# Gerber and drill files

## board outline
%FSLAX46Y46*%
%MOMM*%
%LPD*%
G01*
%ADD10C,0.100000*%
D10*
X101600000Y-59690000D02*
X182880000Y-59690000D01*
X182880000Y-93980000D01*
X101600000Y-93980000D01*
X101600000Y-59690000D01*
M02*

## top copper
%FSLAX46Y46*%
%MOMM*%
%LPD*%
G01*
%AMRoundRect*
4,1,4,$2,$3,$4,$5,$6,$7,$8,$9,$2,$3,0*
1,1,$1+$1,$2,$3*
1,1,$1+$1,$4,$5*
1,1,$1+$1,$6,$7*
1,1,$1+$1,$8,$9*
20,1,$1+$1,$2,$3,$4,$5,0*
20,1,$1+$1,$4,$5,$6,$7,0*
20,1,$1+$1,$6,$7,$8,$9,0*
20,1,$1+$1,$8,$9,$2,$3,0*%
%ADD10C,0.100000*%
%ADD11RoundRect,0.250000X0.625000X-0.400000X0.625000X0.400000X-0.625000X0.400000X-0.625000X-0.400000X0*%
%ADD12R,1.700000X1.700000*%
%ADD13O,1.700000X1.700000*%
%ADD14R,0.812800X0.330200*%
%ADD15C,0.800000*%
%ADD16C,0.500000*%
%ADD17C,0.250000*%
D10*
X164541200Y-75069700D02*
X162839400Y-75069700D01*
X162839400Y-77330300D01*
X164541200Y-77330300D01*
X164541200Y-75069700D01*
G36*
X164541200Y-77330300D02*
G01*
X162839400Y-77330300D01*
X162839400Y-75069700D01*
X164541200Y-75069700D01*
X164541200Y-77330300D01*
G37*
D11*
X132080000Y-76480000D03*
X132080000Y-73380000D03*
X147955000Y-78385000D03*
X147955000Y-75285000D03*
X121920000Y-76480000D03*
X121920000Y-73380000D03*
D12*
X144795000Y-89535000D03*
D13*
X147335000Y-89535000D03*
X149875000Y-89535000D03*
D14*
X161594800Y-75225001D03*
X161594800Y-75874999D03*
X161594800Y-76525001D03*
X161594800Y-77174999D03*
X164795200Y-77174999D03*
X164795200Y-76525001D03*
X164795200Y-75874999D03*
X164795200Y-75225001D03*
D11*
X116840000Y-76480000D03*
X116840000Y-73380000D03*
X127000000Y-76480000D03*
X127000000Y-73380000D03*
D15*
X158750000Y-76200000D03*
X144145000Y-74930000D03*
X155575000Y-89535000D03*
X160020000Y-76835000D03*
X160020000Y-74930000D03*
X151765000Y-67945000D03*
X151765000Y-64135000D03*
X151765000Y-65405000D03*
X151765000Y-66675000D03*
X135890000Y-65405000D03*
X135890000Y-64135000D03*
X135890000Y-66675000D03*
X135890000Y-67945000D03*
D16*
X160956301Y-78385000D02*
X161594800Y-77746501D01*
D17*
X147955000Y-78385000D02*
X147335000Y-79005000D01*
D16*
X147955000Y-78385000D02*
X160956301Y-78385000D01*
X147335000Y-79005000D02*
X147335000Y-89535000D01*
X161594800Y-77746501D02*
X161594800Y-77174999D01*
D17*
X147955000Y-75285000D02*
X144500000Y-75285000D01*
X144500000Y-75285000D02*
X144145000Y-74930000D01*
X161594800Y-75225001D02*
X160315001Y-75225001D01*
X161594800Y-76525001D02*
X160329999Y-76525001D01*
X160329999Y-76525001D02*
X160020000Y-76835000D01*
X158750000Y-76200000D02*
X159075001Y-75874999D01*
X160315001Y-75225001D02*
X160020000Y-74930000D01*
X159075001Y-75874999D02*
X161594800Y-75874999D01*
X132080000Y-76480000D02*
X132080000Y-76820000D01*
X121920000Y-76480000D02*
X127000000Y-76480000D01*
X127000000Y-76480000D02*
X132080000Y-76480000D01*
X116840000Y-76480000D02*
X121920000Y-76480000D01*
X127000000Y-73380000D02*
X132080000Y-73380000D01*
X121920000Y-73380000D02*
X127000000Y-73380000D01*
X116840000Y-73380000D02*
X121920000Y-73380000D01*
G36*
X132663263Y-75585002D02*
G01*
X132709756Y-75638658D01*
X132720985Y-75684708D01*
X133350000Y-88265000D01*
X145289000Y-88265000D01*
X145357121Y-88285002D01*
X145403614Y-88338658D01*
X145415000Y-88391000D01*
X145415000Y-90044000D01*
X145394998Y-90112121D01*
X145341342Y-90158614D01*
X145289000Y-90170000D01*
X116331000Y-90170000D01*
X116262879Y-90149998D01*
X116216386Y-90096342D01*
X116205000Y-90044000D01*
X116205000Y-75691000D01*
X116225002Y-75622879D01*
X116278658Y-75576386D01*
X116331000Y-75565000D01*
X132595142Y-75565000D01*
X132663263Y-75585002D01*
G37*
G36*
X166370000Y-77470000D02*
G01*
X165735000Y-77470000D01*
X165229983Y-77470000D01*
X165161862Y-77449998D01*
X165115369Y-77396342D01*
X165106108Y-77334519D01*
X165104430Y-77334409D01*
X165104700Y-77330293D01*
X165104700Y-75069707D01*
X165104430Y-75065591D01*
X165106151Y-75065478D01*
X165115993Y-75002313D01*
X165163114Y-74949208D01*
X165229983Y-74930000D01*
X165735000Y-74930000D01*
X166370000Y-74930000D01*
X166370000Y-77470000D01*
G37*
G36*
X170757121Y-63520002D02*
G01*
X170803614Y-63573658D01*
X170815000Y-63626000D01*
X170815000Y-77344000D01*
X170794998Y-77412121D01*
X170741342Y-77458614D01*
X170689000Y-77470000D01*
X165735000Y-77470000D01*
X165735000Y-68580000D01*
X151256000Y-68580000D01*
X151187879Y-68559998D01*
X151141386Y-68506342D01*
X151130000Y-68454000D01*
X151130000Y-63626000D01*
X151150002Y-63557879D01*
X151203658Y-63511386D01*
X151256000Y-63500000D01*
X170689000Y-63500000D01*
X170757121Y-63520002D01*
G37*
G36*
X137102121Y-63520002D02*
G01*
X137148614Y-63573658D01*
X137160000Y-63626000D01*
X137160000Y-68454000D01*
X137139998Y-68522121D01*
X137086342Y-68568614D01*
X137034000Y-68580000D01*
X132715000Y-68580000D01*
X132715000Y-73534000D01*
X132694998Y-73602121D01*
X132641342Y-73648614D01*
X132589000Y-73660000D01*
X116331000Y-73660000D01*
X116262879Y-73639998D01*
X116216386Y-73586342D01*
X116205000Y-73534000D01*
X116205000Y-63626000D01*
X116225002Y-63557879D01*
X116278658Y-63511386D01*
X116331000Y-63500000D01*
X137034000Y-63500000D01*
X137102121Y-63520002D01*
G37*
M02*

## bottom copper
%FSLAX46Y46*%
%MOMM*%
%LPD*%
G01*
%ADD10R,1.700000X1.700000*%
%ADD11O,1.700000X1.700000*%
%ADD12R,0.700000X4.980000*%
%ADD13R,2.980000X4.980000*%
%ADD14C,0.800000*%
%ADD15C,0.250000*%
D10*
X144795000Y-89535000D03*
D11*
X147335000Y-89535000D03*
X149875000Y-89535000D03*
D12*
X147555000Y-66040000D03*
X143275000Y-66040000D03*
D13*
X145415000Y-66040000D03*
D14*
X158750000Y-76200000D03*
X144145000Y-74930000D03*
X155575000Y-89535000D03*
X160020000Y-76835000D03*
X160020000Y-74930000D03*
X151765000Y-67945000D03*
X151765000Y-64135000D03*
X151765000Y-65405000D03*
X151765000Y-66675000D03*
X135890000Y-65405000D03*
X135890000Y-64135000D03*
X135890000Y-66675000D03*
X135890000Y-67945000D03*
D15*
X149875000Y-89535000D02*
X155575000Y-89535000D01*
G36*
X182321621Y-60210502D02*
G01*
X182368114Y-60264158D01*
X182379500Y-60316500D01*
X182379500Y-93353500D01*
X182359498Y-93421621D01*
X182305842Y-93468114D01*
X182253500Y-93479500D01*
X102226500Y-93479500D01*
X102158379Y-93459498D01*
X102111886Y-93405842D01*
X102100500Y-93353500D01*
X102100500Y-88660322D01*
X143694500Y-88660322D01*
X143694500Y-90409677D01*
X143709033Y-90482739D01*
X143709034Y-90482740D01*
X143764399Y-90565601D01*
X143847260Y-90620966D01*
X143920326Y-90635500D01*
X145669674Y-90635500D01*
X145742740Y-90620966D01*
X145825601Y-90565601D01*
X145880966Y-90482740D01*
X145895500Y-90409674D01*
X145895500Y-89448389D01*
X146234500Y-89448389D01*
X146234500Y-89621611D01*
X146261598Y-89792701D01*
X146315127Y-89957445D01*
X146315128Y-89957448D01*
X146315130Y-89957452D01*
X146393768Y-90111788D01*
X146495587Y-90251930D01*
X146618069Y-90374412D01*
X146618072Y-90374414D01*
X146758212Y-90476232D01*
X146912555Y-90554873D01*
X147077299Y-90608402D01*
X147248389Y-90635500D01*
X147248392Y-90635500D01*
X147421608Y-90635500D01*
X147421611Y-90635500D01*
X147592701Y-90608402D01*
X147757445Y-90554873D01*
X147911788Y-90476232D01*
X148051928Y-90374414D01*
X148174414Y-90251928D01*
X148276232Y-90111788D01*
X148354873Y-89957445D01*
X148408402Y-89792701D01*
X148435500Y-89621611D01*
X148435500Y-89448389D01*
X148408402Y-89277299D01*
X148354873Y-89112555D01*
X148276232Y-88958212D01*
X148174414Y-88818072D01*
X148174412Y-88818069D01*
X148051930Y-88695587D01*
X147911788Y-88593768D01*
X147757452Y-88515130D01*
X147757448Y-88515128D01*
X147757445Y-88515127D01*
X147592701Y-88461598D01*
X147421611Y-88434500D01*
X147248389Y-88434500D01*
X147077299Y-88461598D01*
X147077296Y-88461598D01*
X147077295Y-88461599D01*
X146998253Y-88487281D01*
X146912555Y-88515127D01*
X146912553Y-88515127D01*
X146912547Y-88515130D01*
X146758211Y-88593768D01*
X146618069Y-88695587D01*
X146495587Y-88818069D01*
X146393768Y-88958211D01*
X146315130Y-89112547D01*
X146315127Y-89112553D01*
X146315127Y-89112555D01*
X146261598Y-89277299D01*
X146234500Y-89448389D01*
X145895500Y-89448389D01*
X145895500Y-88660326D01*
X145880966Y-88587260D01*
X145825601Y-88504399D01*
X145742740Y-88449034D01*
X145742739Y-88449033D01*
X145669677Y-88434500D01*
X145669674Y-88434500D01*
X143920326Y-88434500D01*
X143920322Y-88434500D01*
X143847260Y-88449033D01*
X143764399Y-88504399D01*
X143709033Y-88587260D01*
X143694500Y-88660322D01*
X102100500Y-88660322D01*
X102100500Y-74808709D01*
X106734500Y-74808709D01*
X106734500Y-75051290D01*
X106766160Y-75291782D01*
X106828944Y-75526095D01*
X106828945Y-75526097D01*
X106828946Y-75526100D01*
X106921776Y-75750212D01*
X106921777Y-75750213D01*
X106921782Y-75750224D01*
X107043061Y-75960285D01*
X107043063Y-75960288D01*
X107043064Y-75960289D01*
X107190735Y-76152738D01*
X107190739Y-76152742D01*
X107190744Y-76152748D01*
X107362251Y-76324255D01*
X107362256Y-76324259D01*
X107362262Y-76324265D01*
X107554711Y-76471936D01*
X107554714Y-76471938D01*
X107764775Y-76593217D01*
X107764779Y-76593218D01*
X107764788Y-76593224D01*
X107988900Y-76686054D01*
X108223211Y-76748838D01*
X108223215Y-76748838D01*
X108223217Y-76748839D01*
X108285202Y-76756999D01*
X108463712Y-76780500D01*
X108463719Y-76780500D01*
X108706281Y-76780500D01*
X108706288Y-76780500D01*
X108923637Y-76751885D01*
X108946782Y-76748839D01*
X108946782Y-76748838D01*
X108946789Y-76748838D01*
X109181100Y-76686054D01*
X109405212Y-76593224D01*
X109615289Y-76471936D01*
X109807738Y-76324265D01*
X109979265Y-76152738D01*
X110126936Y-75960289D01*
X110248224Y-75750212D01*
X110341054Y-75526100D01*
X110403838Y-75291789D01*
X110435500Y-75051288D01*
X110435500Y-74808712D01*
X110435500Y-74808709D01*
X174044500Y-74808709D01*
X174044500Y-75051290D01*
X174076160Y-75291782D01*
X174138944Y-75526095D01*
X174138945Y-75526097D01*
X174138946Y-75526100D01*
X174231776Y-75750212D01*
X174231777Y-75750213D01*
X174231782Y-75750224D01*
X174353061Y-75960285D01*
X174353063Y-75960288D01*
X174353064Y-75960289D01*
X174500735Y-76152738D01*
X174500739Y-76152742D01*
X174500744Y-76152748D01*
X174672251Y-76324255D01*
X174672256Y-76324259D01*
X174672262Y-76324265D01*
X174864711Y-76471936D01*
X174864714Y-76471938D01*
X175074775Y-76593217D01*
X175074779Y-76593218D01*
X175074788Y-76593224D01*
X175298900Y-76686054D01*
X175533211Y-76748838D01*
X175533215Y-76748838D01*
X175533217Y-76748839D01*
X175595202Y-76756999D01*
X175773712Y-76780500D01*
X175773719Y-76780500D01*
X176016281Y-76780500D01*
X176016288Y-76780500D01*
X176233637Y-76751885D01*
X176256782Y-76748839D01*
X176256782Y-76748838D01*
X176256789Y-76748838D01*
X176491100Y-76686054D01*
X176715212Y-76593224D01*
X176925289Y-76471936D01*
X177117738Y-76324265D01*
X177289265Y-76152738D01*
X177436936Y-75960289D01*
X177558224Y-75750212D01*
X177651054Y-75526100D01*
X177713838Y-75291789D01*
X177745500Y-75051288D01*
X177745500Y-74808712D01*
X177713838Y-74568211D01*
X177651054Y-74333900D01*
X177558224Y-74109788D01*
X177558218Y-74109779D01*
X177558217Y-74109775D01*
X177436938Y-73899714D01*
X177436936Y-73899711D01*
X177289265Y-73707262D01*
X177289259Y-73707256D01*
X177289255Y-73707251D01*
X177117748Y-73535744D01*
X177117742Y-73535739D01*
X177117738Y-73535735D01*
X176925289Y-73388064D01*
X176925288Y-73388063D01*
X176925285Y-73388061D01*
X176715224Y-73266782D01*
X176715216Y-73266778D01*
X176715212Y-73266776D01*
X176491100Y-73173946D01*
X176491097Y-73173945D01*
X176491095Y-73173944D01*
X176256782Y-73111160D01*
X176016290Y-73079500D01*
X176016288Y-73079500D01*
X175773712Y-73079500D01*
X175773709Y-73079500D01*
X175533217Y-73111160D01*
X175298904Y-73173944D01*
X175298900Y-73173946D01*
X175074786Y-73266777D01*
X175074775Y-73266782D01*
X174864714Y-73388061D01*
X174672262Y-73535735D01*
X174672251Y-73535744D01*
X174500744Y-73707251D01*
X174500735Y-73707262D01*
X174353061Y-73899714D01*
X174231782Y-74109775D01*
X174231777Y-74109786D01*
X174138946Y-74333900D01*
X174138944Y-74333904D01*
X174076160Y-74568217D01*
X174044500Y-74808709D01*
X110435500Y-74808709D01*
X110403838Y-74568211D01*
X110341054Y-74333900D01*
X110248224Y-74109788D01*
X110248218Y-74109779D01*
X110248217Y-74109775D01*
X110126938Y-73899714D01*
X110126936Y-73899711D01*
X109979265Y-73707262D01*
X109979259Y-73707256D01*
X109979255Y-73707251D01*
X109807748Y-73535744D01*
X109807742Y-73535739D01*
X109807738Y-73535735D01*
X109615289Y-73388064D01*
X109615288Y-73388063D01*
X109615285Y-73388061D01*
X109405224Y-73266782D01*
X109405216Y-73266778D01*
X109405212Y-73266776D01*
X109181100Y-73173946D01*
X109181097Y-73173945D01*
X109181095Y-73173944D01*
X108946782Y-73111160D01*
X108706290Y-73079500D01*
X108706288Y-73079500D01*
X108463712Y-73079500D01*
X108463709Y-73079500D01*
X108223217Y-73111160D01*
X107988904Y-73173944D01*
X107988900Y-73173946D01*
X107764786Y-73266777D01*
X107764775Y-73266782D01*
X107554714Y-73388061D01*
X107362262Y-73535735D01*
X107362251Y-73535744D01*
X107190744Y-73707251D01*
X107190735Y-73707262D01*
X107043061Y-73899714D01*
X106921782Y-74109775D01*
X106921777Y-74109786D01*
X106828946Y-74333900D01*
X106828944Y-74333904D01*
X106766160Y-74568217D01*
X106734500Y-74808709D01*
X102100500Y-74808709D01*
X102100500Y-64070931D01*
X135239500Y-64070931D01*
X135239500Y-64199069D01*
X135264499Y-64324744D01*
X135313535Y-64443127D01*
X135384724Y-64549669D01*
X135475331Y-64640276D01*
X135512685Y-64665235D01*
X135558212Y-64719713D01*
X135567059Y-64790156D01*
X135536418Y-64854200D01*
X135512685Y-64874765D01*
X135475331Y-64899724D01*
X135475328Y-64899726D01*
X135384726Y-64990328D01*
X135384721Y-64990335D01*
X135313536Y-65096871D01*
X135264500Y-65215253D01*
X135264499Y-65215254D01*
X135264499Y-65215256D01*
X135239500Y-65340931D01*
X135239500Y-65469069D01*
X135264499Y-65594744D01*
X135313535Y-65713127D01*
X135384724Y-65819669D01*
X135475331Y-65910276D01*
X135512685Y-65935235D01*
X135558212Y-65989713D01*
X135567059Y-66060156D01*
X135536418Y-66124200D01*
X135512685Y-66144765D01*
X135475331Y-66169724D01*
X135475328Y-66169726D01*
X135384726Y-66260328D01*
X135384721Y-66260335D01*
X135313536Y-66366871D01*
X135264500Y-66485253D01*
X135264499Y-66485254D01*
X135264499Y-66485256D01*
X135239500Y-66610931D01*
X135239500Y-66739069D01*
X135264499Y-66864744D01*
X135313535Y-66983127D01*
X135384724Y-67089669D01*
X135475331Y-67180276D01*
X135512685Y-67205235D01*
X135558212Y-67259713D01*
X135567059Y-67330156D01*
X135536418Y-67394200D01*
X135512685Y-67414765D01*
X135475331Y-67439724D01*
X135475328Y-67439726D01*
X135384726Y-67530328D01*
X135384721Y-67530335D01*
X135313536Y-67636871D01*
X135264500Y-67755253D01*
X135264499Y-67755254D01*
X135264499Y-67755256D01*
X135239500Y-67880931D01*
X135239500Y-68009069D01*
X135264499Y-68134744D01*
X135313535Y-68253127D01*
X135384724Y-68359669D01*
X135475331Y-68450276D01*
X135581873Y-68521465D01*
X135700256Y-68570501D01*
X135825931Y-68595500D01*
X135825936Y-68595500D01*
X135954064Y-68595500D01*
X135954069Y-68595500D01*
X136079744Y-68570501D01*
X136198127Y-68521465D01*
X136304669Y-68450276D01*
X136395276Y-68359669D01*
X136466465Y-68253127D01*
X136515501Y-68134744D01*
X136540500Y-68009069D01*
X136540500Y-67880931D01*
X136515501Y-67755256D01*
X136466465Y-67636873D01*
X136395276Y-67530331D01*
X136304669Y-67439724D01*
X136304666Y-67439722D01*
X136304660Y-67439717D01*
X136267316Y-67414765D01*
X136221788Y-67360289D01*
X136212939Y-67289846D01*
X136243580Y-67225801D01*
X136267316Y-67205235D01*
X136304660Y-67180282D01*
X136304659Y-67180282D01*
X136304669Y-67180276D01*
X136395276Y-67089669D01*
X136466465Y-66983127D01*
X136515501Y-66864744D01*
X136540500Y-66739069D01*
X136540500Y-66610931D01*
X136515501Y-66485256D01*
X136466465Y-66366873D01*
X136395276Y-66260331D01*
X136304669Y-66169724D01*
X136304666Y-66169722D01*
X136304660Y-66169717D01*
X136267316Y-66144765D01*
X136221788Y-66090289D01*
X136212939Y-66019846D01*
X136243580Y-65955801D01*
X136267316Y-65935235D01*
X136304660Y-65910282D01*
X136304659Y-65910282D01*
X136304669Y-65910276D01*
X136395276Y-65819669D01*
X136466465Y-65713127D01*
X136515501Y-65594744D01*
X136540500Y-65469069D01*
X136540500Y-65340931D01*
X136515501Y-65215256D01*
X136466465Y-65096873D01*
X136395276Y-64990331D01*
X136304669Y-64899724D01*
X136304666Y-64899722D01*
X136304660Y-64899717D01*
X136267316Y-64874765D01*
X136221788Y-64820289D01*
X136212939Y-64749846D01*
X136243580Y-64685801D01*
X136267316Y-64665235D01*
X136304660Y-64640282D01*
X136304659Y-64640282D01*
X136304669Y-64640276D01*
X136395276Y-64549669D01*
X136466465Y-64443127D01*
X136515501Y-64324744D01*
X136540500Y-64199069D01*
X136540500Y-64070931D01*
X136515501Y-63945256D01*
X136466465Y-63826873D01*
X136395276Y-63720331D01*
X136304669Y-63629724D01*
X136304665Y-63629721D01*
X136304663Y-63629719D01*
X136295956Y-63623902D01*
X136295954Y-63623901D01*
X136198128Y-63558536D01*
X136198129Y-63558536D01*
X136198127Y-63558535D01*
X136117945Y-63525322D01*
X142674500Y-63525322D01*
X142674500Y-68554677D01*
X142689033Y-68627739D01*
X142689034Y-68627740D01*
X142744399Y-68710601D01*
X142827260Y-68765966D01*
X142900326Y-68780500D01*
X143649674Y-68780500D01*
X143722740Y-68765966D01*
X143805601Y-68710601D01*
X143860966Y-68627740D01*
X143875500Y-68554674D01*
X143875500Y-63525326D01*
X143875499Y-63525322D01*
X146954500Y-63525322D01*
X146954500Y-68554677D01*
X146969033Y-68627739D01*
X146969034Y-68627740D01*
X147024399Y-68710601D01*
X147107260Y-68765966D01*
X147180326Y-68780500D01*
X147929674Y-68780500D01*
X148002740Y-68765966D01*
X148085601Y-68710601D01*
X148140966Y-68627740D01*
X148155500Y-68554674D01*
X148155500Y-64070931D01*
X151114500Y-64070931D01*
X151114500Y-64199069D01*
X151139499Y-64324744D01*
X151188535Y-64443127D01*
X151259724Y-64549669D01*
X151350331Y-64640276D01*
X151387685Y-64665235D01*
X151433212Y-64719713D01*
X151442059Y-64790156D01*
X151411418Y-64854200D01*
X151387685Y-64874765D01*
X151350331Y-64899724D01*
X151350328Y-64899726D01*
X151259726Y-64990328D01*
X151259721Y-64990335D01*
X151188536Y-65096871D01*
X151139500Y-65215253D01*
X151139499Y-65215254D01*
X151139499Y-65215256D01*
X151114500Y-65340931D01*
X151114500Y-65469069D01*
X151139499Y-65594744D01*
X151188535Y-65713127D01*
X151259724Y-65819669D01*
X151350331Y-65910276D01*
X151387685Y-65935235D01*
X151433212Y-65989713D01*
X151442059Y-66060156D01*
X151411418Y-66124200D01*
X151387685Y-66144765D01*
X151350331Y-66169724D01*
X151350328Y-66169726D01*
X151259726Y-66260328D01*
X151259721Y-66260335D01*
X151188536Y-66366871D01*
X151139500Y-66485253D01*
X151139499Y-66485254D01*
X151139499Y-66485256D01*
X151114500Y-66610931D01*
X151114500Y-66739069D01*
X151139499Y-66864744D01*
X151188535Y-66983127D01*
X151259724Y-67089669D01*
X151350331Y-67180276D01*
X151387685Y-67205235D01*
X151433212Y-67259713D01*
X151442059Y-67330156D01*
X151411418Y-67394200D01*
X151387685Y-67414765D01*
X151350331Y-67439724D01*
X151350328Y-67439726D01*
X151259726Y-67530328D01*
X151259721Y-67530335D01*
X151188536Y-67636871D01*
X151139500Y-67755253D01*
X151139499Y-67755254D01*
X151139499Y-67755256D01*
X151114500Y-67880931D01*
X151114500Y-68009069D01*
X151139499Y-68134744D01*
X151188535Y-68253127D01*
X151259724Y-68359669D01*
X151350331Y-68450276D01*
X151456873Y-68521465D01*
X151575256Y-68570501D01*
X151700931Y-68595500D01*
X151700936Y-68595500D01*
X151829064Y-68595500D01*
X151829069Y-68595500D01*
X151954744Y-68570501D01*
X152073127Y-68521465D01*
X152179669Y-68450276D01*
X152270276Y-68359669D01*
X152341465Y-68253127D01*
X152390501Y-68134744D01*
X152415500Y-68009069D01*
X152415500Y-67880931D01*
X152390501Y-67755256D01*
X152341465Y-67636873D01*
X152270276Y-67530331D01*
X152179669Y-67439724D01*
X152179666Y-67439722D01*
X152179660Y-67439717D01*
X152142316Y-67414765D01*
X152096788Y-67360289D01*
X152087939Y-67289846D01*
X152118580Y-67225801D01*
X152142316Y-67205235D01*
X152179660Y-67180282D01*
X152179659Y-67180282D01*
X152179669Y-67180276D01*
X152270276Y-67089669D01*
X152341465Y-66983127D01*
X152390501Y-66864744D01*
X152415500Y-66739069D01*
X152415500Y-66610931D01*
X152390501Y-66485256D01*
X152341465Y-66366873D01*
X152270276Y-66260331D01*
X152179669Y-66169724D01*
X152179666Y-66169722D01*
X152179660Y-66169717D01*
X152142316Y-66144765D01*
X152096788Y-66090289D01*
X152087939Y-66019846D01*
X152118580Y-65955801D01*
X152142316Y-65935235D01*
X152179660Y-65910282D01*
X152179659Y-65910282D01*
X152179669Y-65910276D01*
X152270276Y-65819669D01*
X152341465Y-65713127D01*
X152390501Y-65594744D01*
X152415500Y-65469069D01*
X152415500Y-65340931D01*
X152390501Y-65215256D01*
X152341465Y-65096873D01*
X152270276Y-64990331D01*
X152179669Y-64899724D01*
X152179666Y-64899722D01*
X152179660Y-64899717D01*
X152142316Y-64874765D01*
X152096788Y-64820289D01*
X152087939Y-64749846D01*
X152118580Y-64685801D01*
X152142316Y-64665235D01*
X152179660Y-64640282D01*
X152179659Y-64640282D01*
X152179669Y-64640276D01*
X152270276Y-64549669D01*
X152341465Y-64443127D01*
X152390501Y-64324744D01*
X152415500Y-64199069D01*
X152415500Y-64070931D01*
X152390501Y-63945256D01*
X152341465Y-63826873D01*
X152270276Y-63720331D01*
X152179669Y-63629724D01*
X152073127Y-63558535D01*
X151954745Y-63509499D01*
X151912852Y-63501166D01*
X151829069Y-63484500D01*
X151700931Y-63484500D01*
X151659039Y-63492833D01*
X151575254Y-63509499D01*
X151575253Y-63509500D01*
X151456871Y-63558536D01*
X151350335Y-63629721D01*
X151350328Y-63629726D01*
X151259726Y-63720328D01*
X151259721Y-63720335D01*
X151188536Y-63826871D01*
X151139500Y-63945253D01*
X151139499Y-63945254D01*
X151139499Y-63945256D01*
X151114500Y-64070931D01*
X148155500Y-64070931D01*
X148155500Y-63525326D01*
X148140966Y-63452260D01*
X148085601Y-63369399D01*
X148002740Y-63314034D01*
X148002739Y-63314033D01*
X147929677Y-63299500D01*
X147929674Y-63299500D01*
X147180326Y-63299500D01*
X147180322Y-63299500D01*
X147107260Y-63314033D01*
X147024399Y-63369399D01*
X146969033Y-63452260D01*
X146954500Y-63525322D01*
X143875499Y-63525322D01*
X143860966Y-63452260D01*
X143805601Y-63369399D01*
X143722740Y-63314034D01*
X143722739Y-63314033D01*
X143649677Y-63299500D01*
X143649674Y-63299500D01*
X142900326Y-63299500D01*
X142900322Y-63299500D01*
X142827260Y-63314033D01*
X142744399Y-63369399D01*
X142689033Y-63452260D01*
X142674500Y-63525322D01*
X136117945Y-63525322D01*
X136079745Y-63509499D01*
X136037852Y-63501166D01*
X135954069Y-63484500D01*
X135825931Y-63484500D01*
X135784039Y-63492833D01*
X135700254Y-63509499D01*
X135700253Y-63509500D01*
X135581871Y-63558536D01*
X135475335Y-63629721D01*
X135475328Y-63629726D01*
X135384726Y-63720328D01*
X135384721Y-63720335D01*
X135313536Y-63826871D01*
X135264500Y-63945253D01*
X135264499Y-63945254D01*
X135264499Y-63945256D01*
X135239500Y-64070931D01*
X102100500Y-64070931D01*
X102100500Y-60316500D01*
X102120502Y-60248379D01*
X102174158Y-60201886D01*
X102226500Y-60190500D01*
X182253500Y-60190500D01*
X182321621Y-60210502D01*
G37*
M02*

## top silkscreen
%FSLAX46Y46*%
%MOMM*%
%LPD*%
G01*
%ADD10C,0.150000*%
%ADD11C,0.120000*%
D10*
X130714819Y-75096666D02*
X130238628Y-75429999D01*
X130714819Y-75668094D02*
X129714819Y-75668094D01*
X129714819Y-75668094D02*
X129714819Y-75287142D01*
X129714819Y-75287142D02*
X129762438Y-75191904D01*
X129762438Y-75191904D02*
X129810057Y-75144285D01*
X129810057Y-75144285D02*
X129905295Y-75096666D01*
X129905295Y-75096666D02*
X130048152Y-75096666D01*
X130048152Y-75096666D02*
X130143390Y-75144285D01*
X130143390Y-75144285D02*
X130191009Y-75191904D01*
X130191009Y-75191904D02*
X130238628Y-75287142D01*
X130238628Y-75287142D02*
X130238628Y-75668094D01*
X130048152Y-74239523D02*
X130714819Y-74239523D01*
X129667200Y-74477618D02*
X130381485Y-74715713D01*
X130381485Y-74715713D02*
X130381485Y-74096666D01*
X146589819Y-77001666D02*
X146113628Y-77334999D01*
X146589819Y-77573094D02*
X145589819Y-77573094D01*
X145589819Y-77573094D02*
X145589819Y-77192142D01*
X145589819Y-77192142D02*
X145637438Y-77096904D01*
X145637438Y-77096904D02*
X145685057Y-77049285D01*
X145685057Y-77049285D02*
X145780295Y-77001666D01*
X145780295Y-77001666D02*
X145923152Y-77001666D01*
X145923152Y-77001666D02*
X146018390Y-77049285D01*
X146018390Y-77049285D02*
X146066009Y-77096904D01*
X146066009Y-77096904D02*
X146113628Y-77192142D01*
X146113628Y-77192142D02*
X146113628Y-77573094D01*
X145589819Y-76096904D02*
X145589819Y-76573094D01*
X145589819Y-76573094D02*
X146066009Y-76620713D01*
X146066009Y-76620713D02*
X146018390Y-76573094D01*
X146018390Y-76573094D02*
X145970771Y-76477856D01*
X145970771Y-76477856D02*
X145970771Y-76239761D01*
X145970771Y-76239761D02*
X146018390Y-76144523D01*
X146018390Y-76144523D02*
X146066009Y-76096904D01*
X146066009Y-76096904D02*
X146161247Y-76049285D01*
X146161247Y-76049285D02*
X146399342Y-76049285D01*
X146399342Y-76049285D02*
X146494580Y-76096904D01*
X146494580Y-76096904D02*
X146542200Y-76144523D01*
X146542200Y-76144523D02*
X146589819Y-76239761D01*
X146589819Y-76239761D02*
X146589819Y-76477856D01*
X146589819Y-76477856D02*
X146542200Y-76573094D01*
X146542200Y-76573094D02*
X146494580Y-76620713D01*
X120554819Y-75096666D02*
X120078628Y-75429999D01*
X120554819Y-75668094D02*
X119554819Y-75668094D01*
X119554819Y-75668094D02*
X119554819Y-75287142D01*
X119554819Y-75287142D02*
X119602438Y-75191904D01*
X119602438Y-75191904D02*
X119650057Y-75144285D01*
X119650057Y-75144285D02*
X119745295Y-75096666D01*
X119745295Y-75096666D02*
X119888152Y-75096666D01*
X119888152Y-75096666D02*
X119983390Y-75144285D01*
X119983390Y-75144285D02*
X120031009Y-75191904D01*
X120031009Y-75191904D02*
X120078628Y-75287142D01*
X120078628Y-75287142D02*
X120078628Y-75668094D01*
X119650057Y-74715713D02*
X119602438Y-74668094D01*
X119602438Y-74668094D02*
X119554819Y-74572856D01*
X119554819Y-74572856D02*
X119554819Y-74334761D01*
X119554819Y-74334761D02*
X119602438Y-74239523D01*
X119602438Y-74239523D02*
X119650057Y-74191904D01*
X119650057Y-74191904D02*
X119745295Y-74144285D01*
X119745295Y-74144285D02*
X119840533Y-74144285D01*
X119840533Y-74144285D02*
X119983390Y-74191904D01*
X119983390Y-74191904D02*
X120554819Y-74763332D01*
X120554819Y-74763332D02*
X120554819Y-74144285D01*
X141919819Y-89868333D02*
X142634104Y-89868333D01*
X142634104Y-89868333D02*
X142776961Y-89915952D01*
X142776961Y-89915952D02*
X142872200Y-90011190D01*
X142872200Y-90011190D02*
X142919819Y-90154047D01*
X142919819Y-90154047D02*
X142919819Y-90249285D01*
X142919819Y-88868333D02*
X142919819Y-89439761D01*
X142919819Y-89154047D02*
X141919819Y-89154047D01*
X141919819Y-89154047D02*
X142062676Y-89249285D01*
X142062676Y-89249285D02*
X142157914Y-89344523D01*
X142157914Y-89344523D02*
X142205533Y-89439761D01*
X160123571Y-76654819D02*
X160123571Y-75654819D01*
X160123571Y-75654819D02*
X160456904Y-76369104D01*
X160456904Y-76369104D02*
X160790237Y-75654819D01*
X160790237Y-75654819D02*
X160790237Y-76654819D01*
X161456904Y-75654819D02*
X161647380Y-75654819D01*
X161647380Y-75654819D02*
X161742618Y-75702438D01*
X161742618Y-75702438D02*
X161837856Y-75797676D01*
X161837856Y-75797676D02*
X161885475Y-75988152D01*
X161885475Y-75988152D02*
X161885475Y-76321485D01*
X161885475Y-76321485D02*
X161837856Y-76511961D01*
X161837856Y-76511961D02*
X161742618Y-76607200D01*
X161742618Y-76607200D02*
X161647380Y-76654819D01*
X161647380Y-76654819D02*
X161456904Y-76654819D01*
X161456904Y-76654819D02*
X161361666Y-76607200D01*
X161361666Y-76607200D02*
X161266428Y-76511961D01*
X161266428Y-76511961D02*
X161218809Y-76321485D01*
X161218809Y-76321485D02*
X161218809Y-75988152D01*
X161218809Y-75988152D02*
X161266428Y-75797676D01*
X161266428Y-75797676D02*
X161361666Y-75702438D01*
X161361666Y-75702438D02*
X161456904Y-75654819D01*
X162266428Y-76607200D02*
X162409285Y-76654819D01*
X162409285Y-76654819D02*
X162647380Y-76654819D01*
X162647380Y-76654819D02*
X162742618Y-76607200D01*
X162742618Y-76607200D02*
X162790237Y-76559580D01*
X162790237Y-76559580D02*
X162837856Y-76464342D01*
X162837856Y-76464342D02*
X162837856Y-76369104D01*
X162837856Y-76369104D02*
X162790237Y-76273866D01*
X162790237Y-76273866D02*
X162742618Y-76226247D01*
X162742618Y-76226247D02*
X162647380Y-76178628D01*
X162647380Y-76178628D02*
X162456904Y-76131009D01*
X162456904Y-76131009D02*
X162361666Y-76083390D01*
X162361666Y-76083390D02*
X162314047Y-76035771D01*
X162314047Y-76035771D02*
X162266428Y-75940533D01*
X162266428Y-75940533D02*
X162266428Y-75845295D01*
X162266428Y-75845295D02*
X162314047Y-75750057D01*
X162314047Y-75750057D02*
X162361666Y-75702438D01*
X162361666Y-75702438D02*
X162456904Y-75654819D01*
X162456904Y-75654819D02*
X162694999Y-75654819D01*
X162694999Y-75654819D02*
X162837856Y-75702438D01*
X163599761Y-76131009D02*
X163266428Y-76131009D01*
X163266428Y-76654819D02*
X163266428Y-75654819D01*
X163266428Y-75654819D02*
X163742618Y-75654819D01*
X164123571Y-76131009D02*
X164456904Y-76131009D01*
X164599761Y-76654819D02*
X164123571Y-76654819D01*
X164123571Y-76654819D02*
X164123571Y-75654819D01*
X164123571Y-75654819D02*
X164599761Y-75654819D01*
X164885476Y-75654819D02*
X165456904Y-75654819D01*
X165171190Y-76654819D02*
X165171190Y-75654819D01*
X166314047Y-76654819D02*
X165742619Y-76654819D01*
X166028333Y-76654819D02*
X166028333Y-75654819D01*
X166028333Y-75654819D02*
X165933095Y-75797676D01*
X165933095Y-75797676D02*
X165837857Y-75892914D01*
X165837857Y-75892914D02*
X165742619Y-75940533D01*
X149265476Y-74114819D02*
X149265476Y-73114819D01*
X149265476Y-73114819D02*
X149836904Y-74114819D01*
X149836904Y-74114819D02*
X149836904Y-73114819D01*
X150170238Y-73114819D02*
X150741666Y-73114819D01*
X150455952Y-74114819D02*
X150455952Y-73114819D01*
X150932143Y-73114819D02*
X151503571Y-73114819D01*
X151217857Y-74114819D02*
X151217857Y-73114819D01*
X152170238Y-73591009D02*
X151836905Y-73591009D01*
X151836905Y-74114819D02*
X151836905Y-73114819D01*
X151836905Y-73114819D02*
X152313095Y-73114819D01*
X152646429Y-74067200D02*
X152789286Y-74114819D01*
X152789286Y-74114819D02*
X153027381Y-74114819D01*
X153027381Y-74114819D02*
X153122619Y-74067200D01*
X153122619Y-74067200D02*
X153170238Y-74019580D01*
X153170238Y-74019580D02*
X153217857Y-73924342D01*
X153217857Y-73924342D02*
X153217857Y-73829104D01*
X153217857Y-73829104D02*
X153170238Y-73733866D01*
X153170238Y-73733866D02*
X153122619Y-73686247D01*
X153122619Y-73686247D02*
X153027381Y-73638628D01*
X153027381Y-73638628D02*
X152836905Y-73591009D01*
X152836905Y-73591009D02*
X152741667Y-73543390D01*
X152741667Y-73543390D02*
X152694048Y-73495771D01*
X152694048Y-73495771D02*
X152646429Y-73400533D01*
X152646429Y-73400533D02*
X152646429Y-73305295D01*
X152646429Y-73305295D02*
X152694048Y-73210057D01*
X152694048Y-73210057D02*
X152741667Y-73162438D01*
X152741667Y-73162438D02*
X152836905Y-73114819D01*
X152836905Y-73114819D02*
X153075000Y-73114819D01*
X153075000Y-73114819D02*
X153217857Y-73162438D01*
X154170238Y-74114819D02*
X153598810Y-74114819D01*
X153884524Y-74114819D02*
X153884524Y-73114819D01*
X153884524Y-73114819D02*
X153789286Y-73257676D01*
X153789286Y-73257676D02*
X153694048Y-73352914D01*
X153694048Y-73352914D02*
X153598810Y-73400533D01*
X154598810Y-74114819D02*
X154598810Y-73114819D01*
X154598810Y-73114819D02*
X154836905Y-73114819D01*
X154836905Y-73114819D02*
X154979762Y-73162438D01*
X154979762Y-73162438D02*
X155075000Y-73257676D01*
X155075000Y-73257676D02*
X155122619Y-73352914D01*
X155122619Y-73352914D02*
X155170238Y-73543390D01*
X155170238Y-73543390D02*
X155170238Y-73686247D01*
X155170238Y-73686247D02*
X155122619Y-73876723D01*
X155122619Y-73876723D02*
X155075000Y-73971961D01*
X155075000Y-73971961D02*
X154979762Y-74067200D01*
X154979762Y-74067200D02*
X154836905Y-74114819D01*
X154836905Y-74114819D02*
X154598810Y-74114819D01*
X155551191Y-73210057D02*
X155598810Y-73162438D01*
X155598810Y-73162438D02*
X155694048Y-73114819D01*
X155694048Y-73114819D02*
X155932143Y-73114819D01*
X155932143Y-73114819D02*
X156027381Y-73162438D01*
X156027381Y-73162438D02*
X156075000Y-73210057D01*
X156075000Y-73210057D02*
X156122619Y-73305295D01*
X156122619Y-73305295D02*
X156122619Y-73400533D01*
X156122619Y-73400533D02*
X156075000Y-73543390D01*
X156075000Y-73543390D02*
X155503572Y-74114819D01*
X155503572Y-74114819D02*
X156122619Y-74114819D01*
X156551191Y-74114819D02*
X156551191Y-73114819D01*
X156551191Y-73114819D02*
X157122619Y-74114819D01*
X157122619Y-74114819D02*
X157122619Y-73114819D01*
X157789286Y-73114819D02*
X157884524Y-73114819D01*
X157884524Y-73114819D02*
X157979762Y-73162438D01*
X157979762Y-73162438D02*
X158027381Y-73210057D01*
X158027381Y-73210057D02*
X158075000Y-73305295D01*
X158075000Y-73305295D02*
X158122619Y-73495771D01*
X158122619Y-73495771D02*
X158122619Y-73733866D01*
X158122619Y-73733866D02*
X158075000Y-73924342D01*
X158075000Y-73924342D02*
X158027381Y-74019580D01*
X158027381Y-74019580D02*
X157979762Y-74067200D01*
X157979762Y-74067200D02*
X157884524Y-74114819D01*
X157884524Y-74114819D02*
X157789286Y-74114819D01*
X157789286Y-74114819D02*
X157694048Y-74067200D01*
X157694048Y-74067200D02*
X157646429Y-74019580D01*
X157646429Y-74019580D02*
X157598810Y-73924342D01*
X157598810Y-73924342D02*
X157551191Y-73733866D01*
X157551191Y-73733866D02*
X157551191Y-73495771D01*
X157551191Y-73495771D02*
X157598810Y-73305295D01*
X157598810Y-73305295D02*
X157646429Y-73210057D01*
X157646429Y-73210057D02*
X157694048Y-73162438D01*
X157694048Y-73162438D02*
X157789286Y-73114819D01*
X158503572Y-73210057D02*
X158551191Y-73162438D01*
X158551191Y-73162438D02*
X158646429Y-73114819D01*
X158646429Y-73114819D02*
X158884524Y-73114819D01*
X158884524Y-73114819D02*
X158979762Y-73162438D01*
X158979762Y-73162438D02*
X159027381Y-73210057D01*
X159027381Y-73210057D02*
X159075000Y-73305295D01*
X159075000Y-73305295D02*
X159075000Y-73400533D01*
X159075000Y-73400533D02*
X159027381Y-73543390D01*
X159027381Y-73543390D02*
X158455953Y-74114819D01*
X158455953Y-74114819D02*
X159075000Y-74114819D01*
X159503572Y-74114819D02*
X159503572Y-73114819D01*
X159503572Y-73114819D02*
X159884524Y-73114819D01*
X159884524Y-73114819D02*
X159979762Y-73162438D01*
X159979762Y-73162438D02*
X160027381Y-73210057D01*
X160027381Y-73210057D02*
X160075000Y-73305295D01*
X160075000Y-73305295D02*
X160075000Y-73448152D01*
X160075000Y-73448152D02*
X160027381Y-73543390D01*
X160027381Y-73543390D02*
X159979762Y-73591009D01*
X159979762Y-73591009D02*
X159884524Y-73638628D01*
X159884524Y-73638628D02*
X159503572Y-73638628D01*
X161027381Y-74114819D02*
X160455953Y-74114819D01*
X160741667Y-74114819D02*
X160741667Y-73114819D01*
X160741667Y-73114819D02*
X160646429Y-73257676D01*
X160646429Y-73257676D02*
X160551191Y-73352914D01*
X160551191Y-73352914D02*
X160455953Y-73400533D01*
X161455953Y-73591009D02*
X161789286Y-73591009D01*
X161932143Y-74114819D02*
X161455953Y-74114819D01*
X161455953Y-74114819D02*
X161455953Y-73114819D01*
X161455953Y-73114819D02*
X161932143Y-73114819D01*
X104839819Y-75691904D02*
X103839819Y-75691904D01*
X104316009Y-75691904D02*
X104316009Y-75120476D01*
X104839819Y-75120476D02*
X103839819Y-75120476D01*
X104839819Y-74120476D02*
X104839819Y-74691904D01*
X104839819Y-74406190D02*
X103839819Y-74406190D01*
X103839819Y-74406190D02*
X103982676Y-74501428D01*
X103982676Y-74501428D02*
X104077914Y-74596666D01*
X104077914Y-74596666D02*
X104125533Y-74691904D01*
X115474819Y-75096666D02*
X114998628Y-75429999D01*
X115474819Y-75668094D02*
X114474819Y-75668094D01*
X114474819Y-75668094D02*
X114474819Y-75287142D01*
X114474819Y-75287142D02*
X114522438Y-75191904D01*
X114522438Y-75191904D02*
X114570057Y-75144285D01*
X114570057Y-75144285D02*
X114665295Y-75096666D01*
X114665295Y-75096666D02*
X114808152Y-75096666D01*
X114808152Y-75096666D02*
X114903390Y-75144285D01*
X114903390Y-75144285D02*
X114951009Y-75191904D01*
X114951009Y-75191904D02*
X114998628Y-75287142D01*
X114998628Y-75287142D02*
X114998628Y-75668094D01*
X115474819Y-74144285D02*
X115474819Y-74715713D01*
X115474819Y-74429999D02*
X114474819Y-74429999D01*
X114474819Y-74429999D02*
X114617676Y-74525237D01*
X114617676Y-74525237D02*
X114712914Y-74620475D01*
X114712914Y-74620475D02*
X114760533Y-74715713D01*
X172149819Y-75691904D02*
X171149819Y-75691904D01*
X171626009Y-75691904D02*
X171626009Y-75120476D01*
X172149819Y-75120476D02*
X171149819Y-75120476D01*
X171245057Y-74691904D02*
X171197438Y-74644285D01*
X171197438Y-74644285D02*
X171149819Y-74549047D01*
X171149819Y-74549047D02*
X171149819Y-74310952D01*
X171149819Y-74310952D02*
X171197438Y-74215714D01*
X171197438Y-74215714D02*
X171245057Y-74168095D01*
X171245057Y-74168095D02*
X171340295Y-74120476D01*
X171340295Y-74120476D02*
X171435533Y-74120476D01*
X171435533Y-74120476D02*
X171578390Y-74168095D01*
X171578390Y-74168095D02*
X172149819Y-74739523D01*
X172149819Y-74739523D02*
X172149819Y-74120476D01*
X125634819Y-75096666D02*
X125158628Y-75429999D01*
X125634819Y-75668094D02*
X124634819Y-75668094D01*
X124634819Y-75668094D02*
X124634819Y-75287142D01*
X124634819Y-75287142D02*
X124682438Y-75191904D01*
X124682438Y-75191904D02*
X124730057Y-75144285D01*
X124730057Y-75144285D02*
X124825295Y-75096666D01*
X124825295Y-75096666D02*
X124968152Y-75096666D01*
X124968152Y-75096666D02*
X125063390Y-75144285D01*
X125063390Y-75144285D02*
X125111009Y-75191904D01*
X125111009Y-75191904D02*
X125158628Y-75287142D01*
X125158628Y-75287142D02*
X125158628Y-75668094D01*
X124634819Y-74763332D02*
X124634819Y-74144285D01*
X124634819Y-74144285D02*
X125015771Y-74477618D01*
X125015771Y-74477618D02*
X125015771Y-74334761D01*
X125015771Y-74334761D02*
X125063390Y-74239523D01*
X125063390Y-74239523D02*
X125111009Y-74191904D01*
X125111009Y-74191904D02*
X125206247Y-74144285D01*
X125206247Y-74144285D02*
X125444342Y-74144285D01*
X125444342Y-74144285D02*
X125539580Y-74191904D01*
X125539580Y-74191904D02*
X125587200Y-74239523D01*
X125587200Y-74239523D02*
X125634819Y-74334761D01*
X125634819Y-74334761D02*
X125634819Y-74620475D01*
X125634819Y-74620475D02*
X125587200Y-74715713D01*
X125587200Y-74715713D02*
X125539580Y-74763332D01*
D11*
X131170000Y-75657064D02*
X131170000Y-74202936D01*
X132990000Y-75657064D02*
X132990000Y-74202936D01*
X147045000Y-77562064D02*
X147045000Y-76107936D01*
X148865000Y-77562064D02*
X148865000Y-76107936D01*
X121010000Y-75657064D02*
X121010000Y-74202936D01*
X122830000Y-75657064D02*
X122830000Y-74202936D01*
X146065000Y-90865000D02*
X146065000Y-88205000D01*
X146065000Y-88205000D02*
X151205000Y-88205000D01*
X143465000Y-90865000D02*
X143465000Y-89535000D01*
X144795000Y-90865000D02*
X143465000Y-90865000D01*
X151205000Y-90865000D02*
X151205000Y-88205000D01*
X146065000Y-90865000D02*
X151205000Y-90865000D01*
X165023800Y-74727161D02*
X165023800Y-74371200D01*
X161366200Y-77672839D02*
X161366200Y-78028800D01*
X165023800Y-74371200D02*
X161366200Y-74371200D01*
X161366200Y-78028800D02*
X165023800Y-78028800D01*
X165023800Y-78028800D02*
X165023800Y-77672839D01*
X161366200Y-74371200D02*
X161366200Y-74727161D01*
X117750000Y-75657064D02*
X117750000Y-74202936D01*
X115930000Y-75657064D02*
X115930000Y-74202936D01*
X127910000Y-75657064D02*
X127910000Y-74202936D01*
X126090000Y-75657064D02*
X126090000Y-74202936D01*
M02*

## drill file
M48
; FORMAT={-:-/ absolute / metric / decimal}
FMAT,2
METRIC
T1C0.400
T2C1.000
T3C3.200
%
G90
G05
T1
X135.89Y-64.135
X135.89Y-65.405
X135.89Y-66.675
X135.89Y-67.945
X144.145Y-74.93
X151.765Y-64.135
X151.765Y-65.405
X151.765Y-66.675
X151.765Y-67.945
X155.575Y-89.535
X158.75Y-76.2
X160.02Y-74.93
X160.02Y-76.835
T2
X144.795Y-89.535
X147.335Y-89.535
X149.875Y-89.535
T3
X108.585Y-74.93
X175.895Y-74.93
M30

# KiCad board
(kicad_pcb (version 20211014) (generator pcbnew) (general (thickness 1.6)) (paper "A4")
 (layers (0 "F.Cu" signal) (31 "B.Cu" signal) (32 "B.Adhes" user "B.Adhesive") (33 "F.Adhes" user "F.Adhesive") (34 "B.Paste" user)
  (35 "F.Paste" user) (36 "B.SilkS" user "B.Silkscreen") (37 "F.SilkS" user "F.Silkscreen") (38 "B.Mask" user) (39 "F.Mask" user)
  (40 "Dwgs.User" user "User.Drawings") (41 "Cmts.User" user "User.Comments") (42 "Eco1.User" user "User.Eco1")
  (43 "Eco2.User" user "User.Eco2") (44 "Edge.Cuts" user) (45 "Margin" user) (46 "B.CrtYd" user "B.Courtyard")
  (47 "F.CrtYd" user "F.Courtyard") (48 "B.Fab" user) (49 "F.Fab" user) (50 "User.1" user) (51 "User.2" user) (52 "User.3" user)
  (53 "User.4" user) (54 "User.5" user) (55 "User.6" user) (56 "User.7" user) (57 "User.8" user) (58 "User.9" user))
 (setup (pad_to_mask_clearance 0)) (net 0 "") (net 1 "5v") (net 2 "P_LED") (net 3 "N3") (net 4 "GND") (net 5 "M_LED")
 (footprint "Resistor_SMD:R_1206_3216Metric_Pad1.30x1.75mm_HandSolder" (layer "F.Cu") (at 132.08 74.93 90)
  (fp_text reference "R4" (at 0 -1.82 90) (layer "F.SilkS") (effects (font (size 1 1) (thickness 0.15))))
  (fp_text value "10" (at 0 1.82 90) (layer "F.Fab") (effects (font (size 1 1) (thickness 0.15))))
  (fp_line (start -0.727064 -0.91) (end 0.727064 -0.91) (layer "F.SilkS") (width 0.12))
  (fp_line (start -0.727064 0.91) (end 0.727064 0.91) (layer "F.SilkS") (width 0.12))
  (pad "1" smd roundrect (at -1.55 0 90) (size 1.3 1.75) (layers "F.Cu" "F.Paste" "F.Mask") (roundrect_rratio 0.1923076923) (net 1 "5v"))
  (pad "2" smd roundrect (at 1.55 0 90) (size 1.3 1.75) (layers "F.Cu" "F.Paste" "F.Mask") (roundrect_rratio 0.1923076923) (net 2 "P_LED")))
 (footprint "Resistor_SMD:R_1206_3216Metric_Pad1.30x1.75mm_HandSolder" (layer "F.Cu") (at 147.955 76.835 90)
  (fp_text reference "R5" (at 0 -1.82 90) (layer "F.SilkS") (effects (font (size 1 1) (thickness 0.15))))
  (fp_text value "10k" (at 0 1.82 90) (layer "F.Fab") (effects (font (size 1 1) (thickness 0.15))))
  (fp_line (start -0.727064 -0.91) (end 0.727064 -0.91) (layer "F.SilkS") (width 0.12))
  (fp_line (start -0.727064 0.91) (end 0.727064 0.91) (layer "F.SilkS") (width 0.12))
  (pad "1" smd roundrect (at -1.55 0 90) (size 1.3 1.75) (layers "F.Cu" "F.Paste" "F.Mask") (roundrect_rratio 0.1923076923) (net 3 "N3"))
  (pad "2" smd roundrect (at 1.55 0 90) (size 1.3 1.75) (layers "F.Cu" "F.Paste" "F.Mask") (roundrect_rratio 0.1923076923) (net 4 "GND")))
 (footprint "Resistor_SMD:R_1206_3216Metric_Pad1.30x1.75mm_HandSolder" (layer "F.Cu") (at 121.92 74.93 90)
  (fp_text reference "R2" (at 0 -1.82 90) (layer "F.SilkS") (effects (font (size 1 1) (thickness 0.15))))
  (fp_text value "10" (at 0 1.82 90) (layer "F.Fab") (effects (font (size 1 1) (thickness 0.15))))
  (fp_line (start -0.727064 -0.91) (end 0.727064 -0.91) (layer "F.SilkS") (width 0.12))
  (fp_line (start -0.727064 0.91) (end 0.727064 0.91) (layer "F.SilkS") (width 0.12))
  (pad "1" smd roundrect (at -1.55 0 90) (size 1.3 1.75) (layers "F.Cu" "F.Paste" "F.Mask") (roundrect_rratio 0.1923076923) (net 1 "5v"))
  (pad "2" smd roundrect (at 1.55 0 90) (size 1.3 1.75) (layers "F.Cu" "F.Paste" "F.Mask") (roundrect_rratio 0.1923076923) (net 2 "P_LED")))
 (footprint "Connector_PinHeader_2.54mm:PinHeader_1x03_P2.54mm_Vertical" (layer "F.Cu") (at 144.795 89.535 90)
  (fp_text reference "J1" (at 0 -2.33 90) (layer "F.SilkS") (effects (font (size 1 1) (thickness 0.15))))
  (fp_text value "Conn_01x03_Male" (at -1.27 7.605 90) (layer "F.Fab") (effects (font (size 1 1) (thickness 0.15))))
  (fp_line (start -1.33 1.27) (end 1.33 1.27) (layer "F.SilkS") (width 0.12))
  (fp_line (start 1.33 1.27) (end 1.33 6.41) (layer "F.SilkS") (width 0.12))
  (fp_line (start -1.33 -1.33) (end 0 -1.33) (layer "F.SilkS") (width 0.12))
  (fp_line (start -1.33 0) (end -1.33 -1.33) (layer "F.SilkS") (width 0.12))
  (fp_line (start -1.33 6.41) (end 1.33 6.41) (layer "F.SilkS") (width 0.12))
  (fp_line (start -1.33 1.27) (end -1.33 6.41) (layer "F.SilkS") (width 0.12))
  (pad "1" thru_hole rect (at 0 0 90) (size 1.7 1.7) (drill 1) (layers *.Cu *.Mask) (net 1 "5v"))
  (pad "2" thru_hole oval (at 0 2.54 90) (size 1.7 1.7) (drill 1) (layers *.Cu *.Mask) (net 3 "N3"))
  (pad "3" thru_hole oval (at 0 5.08 90) (size 1.7 1.7) (drill 1) (layers *.Cu *.Mask) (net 4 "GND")))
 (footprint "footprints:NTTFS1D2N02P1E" (layer "F.Cu") (at 163.195 76.2)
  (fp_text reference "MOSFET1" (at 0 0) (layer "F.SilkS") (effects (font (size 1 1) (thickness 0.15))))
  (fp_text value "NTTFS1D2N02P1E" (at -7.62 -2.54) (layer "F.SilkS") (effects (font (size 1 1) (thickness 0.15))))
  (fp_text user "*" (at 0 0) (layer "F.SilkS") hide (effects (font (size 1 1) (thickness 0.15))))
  (fp_poly (pts (xy 1.3462 -1.1303) (xy -0.3556 -1.1303) (xy -0.3556 1.1303) (xy 1.3462 1.1303)) (layer "F.Cu") (width 0.1) (fill solid))
  (fp_line (start 1.8288 -1.472839) (end 1.8288 -1.8288) (layer "F.SilkS") (width 0.12))
  (fp_line (start -1.8288 1.472839) (end -1.8288 1.8288) (layer "F.SilkS") (width 0.12))
  (fp_line (start 1.8288 -1.8288) (end -1.8288 -1.8288) (layer "F.SilkS") (width 0.12))
  (fp_line (start -1.8288 1.8288) (end 1.8288 1.8288) (layer "F.SilkS") (width 0.12))
  (fp_line (start 1.8288 1.8288) (end 1.8288 1.472839) (layer "F.SilkS") (width 0.12))
  (fp_line (start -1.8288 -1.8288) (end -1.8288 -1.472839) (layer "F.SilkS") (width 0.12))
  (pad "1" smd rect (at -1.6002 -0.974999) (size 0.8128 0.3302) (layers "F.Cu" "F.Paste" "F.Mask") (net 4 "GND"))
  (pad "2" smd rect (at -1.6002 -0.325001) (size 0.8128 0.3302) (layers "F.Cu" "F.Paste" "F.Mask") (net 4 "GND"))
  (pad "3" smd rect (at -1.6002 0.325001) (size 0.8128 0.3302) (layers "F.Cu" "F.Paste" "F.Mask") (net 4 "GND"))
  (pad "4" smd rect (at -1.6002 0.974999) (size 0.8128 0.3302) (layers "F.Cu" "F.Paste" "F.Mask") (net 3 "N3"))
  (pad "5" smd rect (at 1.6002 0.974999) (size 0.8128 0.3302) (layers "F.Cu" "F.Paste" "F.Mask") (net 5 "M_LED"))
  (pad "6" smd rect (at 1.6002 0.325001) (size 0.8128 0.3302) (layers "F.Cu" "F.Paste" "F.Mask") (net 5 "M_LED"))
  (pad "7" smd rect (at 1.6002 -0.325001) (size 0.8128 0.3302) (layers "F.Cu" "F.Paste" "F.Mask") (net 5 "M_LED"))
  (pad "8" smd rect (at 1.6002 -0.974999) (size 0.8128 0.3302) (layers "F.Cu" "F.Paste" "F.Mask") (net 5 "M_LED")))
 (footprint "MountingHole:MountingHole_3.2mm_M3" (layer "F.Cu") (at 108.585 74.93 90)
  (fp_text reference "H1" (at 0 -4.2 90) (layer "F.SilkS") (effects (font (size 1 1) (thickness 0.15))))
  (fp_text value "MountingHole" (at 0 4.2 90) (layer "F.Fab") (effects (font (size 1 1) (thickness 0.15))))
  (pad "" np_thru_hole circle (at 0 0 90) (size 3.2 3.2) (drill 3.2) (layers *.Cu *.Mask)))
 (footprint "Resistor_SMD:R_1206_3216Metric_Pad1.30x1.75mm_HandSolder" (layer "F.Cu") (at 116.84 74.93 90)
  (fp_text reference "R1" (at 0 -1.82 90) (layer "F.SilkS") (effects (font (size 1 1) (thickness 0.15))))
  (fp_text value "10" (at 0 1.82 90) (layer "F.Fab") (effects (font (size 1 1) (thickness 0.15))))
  (fp_line (start -0.727064 0.91) (end 0.727064 0.91) (layer "F.SilkS") (width 0.12))
  (fp_line (start -0.727064 -0.91) (end 0.727064 -0.91) (layer "F.SilkS") (width 0.12))
  (pad "1" smd roundrect (at -1.55 0 90) (size 1.3 1.75) (layers "F.Cu" "F.Paste" "F.Mask") (roundrect_rratio 0.1923076923) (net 1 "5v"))
  (pad "2" smd roundrect (at 1.55 0 90) (size 1.3 1.75) (layers "F.Cu" "F.Paste" "F.Mask") (roundrect_rratio 0.1923076923) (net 2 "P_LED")))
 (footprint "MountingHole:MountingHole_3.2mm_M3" (layer "F.Cu") (at 175.895 74.93 90)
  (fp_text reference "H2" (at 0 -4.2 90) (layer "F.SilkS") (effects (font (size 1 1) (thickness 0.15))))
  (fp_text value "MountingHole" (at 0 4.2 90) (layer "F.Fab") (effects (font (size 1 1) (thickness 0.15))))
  (pad "" np_thru_hole circle (at 0 0 90) (size 3.2 3.2) (drill 3.2) (layers *.Cu *.Mask)))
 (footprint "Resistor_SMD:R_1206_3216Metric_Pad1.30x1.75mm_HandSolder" (layer "F.Cu") (at 127 74.93 90)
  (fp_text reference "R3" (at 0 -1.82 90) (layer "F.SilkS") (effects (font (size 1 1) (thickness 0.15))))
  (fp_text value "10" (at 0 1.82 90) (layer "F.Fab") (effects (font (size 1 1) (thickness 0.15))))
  (fp_line (start -0.727064 0.91) (end 0.727064 0.91) (layer "F.SilkS") (width 0.12))
  (fp_line (start -0.727064 -0.91) (end 0.727064 -0.91) (layer "F.SilkS") (width 0.12))
  (pad "1" smd roundrect (at -1.55 0 90) (size 1.3 1.75) (layers "F.Cu" "F.Paste" "F.Mask") (roundrect_rratio 0.1923076923) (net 1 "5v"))
  (pad "2" smd roundrect (at 1.55 0 90) (size 1.3 1.75) (layers "F.Cu" "F.Paste" "F.Mask") (roundrect_rratio 0.1923076923) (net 2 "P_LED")))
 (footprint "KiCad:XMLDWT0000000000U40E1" (layer "B.Cu") (at 145.415 66.04 180)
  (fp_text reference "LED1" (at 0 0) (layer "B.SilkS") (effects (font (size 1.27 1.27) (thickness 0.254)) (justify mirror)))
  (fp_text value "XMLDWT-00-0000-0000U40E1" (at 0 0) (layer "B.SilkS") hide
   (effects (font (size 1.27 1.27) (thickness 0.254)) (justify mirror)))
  (pad "1" smd rect locked (at -2.14 0 180) (size 0.7 4.98) (layers "B.Cu" "B.Paste" "B.Mask") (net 5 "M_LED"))
  (pad "2" smd rect locked (at 2.14 0 180) (size 0.7 4.98) (layers "B.Cu" "B.Paste" "B.Mask") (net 2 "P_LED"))
  (pad "3" smd rect locked (at 0 0 180) (size 2.98 4.98) (layers "B.Cu" "B.Paste" "B.Mask") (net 4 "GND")))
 (gr_rect (start 101.6 59.69) (end 182.88 93.98) (layer "Edge.Cuts") (width 0.1) (fill none))
 (segment (start 160.956301 78.385) (end 161.5948 77.746501) (width 0.5) (layer "F.Cu") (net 3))
 (segment (start 147.955 78.385) (end 147.335 79.005) (width 0.25) (layer "F.Cu") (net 3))
 (segment (start 147.955 78.385) (end 160.956301 78.385) (width 0.5) (layer "F.Cu") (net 3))
 (segment (start 147.335 79.005) (end 147.335 89.535) (width 0.5) (layer "F.Cu") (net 3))
 (segment (start 161.5948 77.746501) (end 161.5948 77.174999) (width 0.5) (layer "F.Cu") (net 3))
 (segment (start 147.955 75.285) (end 144.5 75.285) (width 0.25) (layer "F.Cu") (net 4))
 (segment (start 144.5 75.285) (end 144.145 74.93) (width 0.25) (layer "F.Cu") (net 4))
 (segment (start 161.5948 75.225001) (end 160.315001 75.225001) (width 0.25) (layer "F.Cu") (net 4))
 (segment (start 161.5948 76.525001) (end 160.329999 76.525001) (width 0.25) (layer "F.Cu") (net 4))
 (segment (start 160.329999 76.525001) (end 160.02 76.835) (width 0.25) (layer "F.Cu") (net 4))
 (segment (start 158.75 76.2) (end 159.075001 75.874999) (width 0.25) (layer "F.Cu") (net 4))
 (segment (start 160.315001 75.225001) (end 160.02 74.93) (width 0.25) (layer "F.Cu") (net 4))
 (segment (start 159.075001 75.874999) (end 161.5948 75.874999) (width 0.25) (layer "F.Cu") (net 4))
 (via (at 158.75 76.2) (size 0.8) (drill 0.4) (layers "F.Cu" "B.Cu") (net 4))
 (via (at 144.145 74.93) (size 0.8) (drill 0.4) (layers "F.Cu" "B.Cu") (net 4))
 (via (at 155.575 89.535) (size 0.8) (drill 0.4) (layers "F.Cu" "B.Cu") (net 4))
 (via (at 160.02 76.835) (size 0.8) (drill 0.4) (layers "F.Cu" "B.Cu") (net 4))
 (via (at 160.02 74.93) (size 0.8) (drill 0.4) (layers "F.Cu" "B.Cu") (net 4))
 (segment (start 149.875 89.535) (end 155.575 89.535) (width 0.25) (layer "B.Cu") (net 4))
 (via (at 151.765 67.945) (size 0.8) (drill 0.4) (layers "F.Cu" "B.Cu") (free) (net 5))
 (via (at 151.765 64.135) (size 0.8) (drill 0.4) (layers "F.Cu" "B.Cu") (free) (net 5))
 (via (at 151.765 65.405) (size 0.8) (drill 0.4) (layers "F.Cu" "B.Cu") (free) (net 5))
 (via (at 151.765 66.675) (size 0.8) (drill 0.4) (layers "F.Cu" "B.Cu") (free) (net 5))
 (segment (start 132.08 76.48) (end 132.08 76.82) (width 0.25) (layer "F.Cu") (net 1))
 (segment (start 121.92 76.48) (end 127 76.48) (width 0.25) (layer "F.Cu") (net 1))
 (segment (start 127 76.48) (end 132.08 76.48) (width 0.25) (layer "F.Cu") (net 1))
 (segment (start 116.84 76.48) (end 121.92 76.48) (width 0.25) (layer "F.Cu") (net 1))
 (segment (start 127 73.38) (end 132.08 73.38) (width 0.25) (layer "F.Cu") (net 2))
 (segment (start 121.92 73.38) (end 127 73.38) (width 0.25) (layer "F.Cu") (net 2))
 (segment (start 116.84 73.38) (end 121.92 73.38) (width 0.25) (layer "F.Cu") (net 2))
 (via (at 135.89 65.405) (size 0.8) (drill 0.4) (layers "F.Cu" "B.Cu") (free) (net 2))
 (via (at 135.89 64.135) (size 0.8) (drill 0.4) (layers "F.Cu" "B.Cu") (free) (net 2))
 (via (at 135.89 66.675) (size 0.8) (drill 0.4) (layers "F.Cu" "B.Cu") (free) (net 2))
 (via (at 135.89 67.945) (size 0.8) (drill 0.4) (layers "F.Cu" "B.Cu") (free) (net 2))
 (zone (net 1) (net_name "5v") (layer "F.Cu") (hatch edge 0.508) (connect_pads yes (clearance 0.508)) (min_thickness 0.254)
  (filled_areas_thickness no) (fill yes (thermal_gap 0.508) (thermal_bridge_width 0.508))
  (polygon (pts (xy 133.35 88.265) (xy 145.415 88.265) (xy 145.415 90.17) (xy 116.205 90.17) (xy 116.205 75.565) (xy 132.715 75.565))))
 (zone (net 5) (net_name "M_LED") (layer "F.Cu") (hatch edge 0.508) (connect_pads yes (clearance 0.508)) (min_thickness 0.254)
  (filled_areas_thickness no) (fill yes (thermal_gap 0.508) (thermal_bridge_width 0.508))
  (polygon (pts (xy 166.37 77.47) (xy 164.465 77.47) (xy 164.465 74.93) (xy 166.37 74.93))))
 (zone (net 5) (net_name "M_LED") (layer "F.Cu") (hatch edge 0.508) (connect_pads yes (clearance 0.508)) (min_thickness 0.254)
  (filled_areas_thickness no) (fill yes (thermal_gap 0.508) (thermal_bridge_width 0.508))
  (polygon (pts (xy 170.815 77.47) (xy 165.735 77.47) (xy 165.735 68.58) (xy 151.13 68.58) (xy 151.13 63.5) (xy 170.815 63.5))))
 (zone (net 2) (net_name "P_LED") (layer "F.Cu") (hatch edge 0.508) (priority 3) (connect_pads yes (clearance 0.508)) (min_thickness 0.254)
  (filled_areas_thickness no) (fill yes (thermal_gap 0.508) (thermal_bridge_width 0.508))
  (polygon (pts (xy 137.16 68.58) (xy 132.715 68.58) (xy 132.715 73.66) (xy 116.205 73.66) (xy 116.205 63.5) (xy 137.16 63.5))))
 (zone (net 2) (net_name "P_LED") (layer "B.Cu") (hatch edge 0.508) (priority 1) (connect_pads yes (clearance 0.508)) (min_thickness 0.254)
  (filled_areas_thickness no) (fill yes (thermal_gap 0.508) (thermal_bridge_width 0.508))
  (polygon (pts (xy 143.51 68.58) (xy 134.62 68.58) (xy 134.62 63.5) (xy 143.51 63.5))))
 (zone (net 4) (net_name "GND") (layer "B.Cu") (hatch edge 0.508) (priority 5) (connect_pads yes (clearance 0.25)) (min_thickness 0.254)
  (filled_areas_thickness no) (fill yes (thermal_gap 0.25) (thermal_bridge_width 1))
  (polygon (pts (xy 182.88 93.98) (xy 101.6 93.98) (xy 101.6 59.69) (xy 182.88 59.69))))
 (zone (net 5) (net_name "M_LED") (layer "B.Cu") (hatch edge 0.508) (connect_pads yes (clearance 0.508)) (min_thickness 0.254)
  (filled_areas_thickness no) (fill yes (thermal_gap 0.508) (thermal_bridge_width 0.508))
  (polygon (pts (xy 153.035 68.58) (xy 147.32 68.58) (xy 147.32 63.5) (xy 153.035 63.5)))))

